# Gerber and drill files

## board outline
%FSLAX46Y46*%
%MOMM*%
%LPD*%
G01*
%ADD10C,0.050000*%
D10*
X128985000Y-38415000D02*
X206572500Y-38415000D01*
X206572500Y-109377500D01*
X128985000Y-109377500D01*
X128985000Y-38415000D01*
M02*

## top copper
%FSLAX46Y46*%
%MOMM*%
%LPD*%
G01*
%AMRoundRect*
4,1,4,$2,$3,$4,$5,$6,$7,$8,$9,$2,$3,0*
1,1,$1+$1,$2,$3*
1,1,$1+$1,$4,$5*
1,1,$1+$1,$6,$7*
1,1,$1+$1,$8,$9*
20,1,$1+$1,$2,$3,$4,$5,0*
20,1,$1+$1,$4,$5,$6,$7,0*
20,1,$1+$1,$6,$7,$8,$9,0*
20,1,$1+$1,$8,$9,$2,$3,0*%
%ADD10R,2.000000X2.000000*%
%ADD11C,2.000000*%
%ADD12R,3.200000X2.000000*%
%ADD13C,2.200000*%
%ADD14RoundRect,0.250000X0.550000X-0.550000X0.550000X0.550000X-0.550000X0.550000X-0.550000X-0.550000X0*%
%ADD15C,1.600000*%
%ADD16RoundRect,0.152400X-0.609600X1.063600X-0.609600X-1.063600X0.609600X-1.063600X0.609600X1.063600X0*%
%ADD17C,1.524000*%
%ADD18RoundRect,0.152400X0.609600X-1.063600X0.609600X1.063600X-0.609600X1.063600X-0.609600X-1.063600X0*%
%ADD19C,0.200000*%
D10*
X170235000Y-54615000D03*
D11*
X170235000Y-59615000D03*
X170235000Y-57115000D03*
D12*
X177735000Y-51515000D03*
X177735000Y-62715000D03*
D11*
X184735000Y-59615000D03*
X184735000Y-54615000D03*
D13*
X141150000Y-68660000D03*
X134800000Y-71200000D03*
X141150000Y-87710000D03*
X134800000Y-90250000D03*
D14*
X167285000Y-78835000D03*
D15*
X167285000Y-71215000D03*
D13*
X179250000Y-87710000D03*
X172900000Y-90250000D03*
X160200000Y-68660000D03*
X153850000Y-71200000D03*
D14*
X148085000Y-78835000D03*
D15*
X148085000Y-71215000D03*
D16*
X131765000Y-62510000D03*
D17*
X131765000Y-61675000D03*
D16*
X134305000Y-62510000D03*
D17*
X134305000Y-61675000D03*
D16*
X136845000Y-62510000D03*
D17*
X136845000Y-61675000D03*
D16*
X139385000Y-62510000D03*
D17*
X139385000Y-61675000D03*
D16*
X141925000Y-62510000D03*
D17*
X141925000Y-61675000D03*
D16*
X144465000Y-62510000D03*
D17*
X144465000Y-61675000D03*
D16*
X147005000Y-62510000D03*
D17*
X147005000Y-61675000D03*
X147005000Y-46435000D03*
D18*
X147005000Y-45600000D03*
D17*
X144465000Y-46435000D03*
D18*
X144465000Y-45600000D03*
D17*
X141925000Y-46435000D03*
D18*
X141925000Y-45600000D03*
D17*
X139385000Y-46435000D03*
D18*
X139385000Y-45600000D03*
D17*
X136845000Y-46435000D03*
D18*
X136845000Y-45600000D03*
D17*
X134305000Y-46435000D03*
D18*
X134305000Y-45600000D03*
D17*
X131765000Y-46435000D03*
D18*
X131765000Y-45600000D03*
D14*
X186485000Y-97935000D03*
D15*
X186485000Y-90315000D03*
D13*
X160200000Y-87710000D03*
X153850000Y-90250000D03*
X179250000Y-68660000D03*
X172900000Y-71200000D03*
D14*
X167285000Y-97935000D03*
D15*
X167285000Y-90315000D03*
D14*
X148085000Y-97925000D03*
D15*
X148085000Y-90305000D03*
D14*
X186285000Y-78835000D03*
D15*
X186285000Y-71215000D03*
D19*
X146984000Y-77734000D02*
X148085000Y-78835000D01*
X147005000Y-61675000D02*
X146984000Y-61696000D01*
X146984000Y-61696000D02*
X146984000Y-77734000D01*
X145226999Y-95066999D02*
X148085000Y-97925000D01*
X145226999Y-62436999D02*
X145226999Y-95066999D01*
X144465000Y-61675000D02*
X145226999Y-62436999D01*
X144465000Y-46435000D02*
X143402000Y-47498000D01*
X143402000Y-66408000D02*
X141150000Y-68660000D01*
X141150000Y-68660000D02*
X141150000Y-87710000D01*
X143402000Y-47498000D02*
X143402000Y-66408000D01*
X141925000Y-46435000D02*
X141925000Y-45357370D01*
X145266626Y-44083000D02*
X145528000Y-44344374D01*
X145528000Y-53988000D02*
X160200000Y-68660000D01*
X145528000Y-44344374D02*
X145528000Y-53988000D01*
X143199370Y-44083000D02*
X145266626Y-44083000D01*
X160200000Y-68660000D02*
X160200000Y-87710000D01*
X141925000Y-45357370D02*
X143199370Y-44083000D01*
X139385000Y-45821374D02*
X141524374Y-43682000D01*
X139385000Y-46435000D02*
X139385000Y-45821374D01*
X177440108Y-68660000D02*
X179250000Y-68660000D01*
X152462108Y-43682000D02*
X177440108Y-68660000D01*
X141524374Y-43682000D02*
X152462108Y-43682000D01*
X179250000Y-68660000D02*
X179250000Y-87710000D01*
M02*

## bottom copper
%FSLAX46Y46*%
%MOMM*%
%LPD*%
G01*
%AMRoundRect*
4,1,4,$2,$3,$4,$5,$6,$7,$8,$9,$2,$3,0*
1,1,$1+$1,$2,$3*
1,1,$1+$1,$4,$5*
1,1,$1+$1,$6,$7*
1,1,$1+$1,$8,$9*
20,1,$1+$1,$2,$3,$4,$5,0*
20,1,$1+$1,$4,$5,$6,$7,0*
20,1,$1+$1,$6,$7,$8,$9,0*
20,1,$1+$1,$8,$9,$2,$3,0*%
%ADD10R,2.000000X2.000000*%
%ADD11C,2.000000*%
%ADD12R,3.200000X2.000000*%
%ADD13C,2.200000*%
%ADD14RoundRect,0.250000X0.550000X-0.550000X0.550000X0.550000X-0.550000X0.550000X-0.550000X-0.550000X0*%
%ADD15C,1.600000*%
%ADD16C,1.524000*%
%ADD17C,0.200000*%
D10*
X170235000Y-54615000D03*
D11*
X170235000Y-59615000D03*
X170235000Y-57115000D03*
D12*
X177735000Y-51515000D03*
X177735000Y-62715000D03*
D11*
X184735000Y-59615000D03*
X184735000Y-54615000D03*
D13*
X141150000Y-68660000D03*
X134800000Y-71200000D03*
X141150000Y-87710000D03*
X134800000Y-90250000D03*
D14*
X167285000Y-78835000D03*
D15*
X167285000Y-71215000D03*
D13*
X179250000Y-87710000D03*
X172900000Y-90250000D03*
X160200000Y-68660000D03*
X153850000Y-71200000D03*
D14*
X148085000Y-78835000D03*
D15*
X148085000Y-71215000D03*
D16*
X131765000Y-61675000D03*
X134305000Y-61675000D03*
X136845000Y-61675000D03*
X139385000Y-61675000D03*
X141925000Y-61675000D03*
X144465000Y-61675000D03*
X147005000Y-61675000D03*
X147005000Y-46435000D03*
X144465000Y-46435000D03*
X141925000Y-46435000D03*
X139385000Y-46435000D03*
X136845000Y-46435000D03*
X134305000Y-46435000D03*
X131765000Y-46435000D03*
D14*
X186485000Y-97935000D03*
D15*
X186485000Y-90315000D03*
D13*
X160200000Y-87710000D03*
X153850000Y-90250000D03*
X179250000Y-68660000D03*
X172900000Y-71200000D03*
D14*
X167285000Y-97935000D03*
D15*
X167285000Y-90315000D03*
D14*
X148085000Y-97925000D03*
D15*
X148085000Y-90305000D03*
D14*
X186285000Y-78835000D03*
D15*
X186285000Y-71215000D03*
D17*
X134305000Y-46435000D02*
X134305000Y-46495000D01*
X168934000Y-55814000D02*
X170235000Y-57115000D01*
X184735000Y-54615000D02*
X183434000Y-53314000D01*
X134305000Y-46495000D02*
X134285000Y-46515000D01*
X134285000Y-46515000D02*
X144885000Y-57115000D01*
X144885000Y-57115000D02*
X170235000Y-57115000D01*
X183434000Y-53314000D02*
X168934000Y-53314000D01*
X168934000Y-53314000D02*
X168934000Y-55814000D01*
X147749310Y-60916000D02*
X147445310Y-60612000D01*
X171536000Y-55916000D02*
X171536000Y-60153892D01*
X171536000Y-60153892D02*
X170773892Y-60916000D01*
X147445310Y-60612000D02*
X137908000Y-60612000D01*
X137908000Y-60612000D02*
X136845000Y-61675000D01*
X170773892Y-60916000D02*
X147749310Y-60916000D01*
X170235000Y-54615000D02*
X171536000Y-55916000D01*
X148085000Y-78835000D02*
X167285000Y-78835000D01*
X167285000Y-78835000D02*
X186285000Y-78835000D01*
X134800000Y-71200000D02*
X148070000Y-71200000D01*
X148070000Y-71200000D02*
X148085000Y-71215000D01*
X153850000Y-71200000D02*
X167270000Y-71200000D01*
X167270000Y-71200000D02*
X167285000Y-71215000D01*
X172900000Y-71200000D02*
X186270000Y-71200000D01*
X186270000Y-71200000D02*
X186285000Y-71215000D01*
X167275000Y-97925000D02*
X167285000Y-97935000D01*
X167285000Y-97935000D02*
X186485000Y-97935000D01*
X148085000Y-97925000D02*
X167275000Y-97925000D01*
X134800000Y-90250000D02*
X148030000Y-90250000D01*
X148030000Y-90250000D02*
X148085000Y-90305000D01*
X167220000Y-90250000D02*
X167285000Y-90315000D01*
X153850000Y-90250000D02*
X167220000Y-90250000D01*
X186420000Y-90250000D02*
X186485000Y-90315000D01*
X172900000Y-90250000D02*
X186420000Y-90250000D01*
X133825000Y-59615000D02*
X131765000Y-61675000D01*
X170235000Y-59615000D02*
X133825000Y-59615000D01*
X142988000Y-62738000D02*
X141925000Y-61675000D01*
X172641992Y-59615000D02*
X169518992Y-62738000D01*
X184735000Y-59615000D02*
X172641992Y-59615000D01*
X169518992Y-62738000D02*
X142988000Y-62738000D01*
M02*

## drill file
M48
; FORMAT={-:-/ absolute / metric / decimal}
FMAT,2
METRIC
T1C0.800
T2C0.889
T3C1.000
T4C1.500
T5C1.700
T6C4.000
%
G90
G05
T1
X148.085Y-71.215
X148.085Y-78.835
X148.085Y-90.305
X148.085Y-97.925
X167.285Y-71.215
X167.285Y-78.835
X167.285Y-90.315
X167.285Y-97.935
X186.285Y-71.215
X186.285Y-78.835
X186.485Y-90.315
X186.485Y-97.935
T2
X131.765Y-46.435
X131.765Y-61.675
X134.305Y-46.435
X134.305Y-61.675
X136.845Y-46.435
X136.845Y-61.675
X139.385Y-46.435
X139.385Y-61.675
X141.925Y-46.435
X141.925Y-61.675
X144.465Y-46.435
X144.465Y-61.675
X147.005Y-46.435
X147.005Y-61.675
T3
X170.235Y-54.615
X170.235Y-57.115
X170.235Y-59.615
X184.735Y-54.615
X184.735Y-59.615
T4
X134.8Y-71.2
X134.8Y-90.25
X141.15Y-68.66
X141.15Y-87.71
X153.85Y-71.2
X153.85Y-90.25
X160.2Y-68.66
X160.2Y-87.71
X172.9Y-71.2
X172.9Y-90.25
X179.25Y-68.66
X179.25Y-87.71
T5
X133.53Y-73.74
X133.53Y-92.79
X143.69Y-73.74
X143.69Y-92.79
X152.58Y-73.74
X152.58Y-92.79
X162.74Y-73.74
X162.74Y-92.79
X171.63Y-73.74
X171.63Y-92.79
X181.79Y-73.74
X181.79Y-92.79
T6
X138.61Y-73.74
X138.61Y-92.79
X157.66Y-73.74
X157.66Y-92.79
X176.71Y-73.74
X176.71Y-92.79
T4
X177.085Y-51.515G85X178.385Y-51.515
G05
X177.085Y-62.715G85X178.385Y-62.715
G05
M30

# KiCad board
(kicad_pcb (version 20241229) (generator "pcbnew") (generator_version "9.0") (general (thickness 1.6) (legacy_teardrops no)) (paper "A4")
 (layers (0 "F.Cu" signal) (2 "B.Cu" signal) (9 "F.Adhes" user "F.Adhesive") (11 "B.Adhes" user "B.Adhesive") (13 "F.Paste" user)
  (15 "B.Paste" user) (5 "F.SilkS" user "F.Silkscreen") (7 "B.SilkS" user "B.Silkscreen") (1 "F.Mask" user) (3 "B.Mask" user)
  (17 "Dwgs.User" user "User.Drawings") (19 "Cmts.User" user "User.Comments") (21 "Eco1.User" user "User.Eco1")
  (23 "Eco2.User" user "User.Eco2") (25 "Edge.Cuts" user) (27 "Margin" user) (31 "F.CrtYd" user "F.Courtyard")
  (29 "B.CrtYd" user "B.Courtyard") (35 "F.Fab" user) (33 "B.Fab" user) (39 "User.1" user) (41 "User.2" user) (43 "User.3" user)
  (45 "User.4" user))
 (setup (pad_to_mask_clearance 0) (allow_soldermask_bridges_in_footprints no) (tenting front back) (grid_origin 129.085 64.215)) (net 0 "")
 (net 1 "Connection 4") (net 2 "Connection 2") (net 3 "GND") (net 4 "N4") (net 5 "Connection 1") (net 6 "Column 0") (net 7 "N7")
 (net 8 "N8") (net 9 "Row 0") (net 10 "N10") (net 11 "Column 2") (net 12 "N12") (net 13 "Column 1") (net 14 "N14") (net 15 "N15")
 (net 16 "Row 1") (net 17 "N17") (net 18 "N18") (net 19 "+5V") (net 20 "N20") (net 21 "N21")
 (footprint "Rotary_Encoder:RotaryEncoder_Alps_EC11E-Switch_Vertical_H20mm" (layer "F.Cu") (at 170.235 54.615)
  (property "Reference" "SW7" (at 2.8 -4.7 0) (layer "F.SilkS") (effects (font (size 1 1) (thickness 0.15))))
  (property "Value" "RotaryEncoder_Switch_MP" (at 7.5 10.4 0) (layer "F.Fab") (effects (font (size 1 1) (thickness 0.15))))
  (pad "A" thru_hole rect (at 0 0) (size 2 2) (drill 1) (layers "*.Cu" "*.Mask") (remove_unused_layers no) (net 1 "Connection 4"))
  (pad "B" thru_hole circle (at 0 5) (size 2 2) (drill 1) (layers "*.Cu" "*.Mask") (remove_unused_layers no) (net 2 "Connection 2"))
  (pad "C" thru_hole circle (at 0 2.5) (size 2 2) (drill 1) (layers "*.Cu" "*.Mask") (remove_unused_layers no) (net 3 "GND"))
  (pad "MP" thru_hole rect (at 7.5 -3.1) (size 3.2 2) (drill oval 2.8 1.5) (layers "*.Cu" "*.Mask") (remove_unused_layers no) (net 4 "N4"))
  (pad "MP" thru_hole rect (at 7.5 8.1) (size 3.2 2) (drill oval 2.8 1.5) (layers "*.Cu" "*.Mask") (remove_unused_layers no) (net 4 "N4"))
  (pad "S1" thru_hole circle (at 14.5 5) (size 2 2) (drill 1) (layers "*.Cu" "*.Mask") (remove_unused_layers no) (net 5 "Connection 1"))
  (pad "S2" thru_hole circle (at 14.5 0) (size 2 2) (drill 1) (layers "*.Cu" "*.Mask") (remove_unused_layers no) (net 3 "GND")))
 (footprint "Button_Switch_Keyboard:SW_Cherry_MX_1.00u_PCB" (layer "F.Cu") (at 141.15 68.66)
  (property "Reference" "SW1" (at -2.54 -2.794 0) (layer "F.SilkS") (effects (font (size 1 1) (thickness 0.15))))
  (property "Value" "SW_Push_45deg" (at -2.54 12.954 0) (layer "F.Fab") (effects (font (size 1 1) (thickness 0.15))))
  (pad "" np_thru_hole circle (at -7.62 5.08) (size 1.7 1.7) (drill 1.7) (layers "*.Cu" "*.Mask"))
  (pad "" np_thru_hole circle (at -2.54 5.08) (size 4 4) (drill 4) (layers "*.Cu" "*.Mask"))
  (pad "" np_thru_hole circle (at 2.54 5.08) (size 1.7 1.7) (drill 1.7) (layers "*.Cu" "*.Mask"))
  (pad "1" thru_hole circle (at 0 0) (size 2.2 2.2) (drill 1.5) (layers "*.Cu" "*.Mask") (remove_unused_layers no) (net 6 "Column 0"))
  (pad "2" thru_hole circle (at -6.35 2.54) (size 2.2 2.2) (drill 1.5) (layers "*.Cu" "*.Mask") (remove_unused_layers no) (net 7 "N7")))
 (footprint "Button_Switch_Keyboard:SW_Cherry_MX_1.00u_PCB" (layer "F.Cu") (at 141.15 87.71)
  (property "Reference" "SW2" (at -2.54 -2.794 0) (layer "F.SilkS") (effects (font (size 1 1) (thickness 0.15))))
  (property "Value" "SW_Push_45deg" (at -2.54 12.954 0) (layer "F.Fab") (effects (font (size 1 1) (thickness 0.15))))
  (pad "" np_thru_hole circle (at -7.62 5.08) (size 1.7 1.7) (drill 1.7) (layers "*.Cu" "*.Mask"))
  (pad "" np_thru_hole circle (at -2.54 5.08) (size 4 4) (drill 4) (layers "*.Cu" "*.Mask"))
  (pad "" np_thru_hole circle (at 2.54 5.08) (size 1.7 1.7) (drill 1.7) (layers "*.Cu" "*.Mask"))
  (pad "1" thru_hole circle (at 0 0) (size 2.2 2.2) (drill 1.5) (layers "*.Cu" "*.Mask") (remove_unused_layers no) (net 6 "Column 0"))
  (pad "2" thru_hole circle (at -6.35 2.54) (size 2.2 2.2) (drill 1.5) (layers "*.Cu" "*.Mask") (remove_unused_layers no) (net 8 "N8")))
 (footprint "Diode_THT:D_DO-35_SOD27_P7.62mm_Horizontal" (layer "F.Cu") (at 167.285 78.835 90)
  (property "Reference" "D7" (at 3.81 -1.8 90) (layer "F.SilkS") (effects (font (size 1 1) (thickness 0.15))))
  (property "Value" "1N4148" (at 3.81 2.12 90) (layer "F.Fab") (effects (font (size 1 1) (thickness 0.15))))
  (pad "1" thru_hole roundrect (at 0 0 90) (size 1.6 1.6) (drill 0.8) (layers "*.Cu" "*.Mask") (remove_unused_layers no)
   (roundrect_rratio 0.15625) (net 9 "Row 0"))
  (pad "2" thru_hole circle (at 7.62 0 90) (size 1.6 1.6) (drill 0.8) (layers "*.Cu" "*.Mask") (remove_unused_layers no) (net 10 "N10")))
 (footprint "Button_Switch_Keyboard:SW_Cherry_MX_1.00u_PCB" (layer "F.Cu") (at 179.25 87.71)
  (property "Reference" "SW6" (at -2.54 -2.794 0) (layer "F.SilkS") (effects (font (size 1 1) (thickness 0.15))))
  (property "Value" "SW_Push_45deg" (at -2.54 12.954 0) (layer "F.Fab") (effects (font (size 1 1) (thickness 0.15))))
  (pad "" np_thru_hole circle (at -7.62 5.08) (size 1.7 1.7) (drill 1.7) (layers "*.Cu" "*.Mask"))
  (pad "" np_thru_hole circle (at -2.54 5.08) (size 4 4) (drill 4) (layers "*.Cu" "*.Mask"))
  (pad "" np_thru_hole circle (at 2.54 5.08) (size 1.7 1.7) (drill 1.7) (layers "*.Cu" "*.Mask"))
  (pad "1" thru_hole circle (at 0 0) (size 2.2 2.2) (drill 1.5) (layers "*.Cu" "*.Mask") (remove_unused_layers no) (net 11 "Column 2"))
  (pad "2" thru_hole circle (at -6.35 2.54) (size 2.2 2.2) (drill 1.5) (layers "*.Cu" "*.Mask") (remove_unused_layers no) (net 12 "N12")))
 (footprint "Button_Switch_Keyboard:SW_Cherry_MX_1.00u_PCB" (layer "F.Cu") (at 160.2 68.66)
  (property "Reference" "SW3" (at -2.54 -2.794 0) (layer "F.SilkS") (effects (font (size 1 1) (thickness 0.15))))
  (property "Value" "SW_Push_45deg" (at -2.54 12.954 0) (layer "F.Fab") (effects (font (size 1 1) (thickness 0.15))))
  (pad "" np_thru_hole circle (at -7.62 5.08) (size 1.7 1.7) (drill 1.7) (layers "*.Cu" "*.Mask"))
  (pad "" np_thru_hole circle (at -2.54 5.08) (size 4 4) (drill 4) (layers "*.Cu" "*.Mask"))
  (pad "" np_thru_hole circle (at 2.54 5.08) (size 1.7 1.7) (drill 1.7) (layers "*.Cu" "*.Mask"))
  (pad "1" thru_hole circle (at 0 0) (size 2.2 2.2) (drill 1.5) (layers "*.Cu" "*.Mask") (remove_unused_layers no) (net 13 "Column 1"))
  (pad "2" thru_hole circle (at -6.35 2.54) (size 2.2 2.2) (drill 1.5) (layers "*.Cu" "*.Mask") (remove_unused_layers no) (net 10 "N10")))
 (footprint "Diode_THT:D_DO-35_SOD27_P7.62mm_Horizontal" (layer "F.Cu") (at 148.085 78.835 90)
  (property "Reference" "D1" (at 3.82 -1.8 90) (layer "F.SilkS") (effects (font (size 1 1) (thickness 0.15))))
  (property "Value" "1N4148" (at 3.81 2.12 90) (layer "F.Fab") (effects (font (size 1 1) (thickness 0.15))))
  (pad "1" thru_hole roundrect (at 0 0 90) (size 1.6 1.6) (drill 0.8) (layers "*.Cu" "*.Mask") (remove_unused_layers no)
   (roundrect_rratio 0.15625) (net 9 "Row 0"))
  (pad "2" thru_hole circle (at 7.62 0 90) (size 1.6 1.6) (drill 0.8) (layers "*.Cu" "*.Mask") (remove_unused_layers no) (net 7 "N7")))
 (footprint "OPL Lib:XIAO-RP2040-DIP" (layer "F.Cu") (at 139.385 54.055 90)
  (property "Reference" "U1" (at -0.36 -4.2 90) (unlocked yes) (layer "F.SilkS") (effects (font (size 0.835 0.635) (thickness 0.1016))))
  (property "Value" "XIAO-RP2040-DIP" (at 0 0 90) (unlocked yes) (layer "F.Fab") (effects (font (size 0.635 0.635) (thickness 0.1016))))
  (pad "1" smd roundrect (at -8.455 -7.62 270) (size 2.432 1.524) (layers "F.Cu" "F.Mask") (roundrect_rratio 0.1) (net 2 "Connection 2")
   (thermal_bridge_angle 45))
  (pad "1" thru_hole circle (at -7.62 -7.62 270) (size 1.524 1.524) (drill 0.889) (layers "*.Cu" "*.Mask") (remove_unused_layers no)
   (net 2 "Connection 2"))
  (pad "2" smd roundrect (at -8.455 -5.08 270) (size 2.432 1.524) (layers "F.Cu" "F.Mask") (roundrect_rratio 0.1) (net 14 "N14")
   (thermal_bridge_angle 45))
  (pad "2" thru_hole circle (at -7.62 -5.08 270) (size 1.524 1.524) (drill 0.889) (layers "*.Cu" "*.Mask") (remove_unused_layers no)
   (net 14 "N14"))
  (pad "3" smd roundrect (at -8.455 -2.54 270) (size 2.432 1.524) (layers "F.Cu" "F.Mask") (roundrect_rratio 0.1) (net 1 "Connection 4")
   (thermal_bridge_angle 45))
  (pad "3" thru_hole circle (at -7.62 -2.54 270) (size 1.524 1.524) (drill 0.889) (layers "*.Cu" "*.Mask") (remove_unused_layers no)
   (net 1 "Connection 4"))
  (pad "4" smd roundrect (at -8.455 0 270) (size 2.432 1.524) (layers "F.Cu" "F.Mask") (roundrect_rratio 0.1) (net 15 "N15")
   (thermal_bridge_angle 45))
  (pad "4" thru_hole circle (at -7.62 0 270) (size 1.524 1.524) (drill 0.889) (layers "*.Cu" "*.Mask") (remove_unused_layers no)
   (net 15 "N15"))
  (pad "5" smd roundrect (at -8.455 2.54 270) (size 2.432 1.524) (layers "F.Cu" "F.Mask") (roundrect_rratio 0.1) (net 5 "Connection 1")
   (thermal_bridge_angle 45))
  (pad "5" thru_hole circle (at -7.62 2.54 270) (size 1.524 1.524) (drill 0.889) (layers "*.Cu" "*.Mask") (remove_unused_layers no)
   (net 5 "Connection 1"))
  (pad "6" smd roundrect (at -8.455 5.08 270) (size 2.432 1.524) (layers "F.Cu" "F.Mask") (roundrect_rratio 0.1) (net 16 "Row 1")
   (thermal_bridge_angle 45))
  (pad "6" thru_hole circle (at -7.62 5.08 270) (size 1.524 1.524) (drill 0.889) (layers "*.Cu" "*.Mask") (remove_unused_layers no)
   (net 16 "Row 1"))
  (pad "7" smd roundrect (at -8.455 7.62 270) (size 2.432 1.524) (layers "F.Cu" "F.Mask") (roundrect_rratio 0.1) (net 9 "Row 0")
   (thermal_bridge_angle 45))
  (pad "7" thru_hole circle (at -7.62 7.62 270) (size 1.524 1.524) (drill 0.889) (layers "*.Cu" "*.Mask") (remove_unused_layers no)
   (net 9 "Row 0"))
  (pad "8" thru_hole circle (at 7.62 7.62 90) (size 1.524 1.524) (drill 0.889) (layers "*.Cu" "*.Mask") (remove_unused_layers no)
   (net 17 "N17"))
  (pad "8" smd roundrect (at 8.455 7.62 90) (size 2.432 1.524) (layers "F.Cu" "F.Mask") (roundrect_rratio 0.1) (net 17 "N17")
   (thermal_bridge_angle 45))
  (pad "9" thru_hole circle (at 7.62 5.08 90) (size 1.524 1.524) (drill 0.889) (layers "*.Cu" "*.Mask") (remove_unused_layers no)
   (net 6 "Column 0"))
  (pad "9" smd roundrect (at 8.455 5.08 90) (size 2.432 1.524) (layers "F.Cu" "F.Mask") (roundrect_rratio 0.1) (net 6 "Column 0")
   (thermal_bridge_angle 45))
  (pad "10" thru_hole circle (at 7.62 2.54 90) (size 1.524 1.524) (drill 0.889) (layers "*.Cu" "*.Mask") (remove_unused_layers no)
   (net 13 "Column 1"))
  (pad "10" smd roundrect (at 8.455 2.54 90) (size 2.432 1.524) (layers "F.Cu" "F.Mask") (roundrect_rratio 0.1) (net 13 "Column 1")
   (thermal_bridge_angle 45))
  (pad "11" thru_hole circle (at 7.62 0 90) (size 1.524 1.524) (drill 0.889) (layers "*.Cu" "*.Mask") (remove_unused_layers no)
   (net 11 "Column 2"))
  (pad "11" smd roundrect (at 8.455 0 90) (size 2.432 1.524) (layers "F.Cu" "F.Mask") (roundrect_rratio 0.1) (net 11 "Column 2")
   (thermal_bridge_angle 45))
  (pad "12" thru_hole circle (at 7.62 -2.54 90) (size 1.524 1.524) (drill 0.889) (layers "*.Cu" "*.Mask") (remove_unused_layers no)
   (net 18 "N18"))
  (pad "12" smd roundrect (at 8.455 -2.54 90) (size 2.432 1.524) (layers "F.Cu" "F.Mask") (roundrect_rratio 0.1) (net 18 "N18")
   (thermal_bridge_angle 45))
  (pad "13" thru_hole circle (at 7.62 -5.08 90) (size 1.524 1.524) (drill 0.889) (layers "*.Cu" "*.Mask") (remove_unused_layers no)
   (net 3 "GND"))
  (pad "13" smd roundrect (at 8.455 -5.08 90) (size 2.432 1.524) (layers "F.Cu" "F.Mask") (roundrect_rratio 0.1) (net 3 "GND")
   (thermal_bridge_angle 45))
  (pad "14" thru_hole circle (at 7.62 -7.62 90) (size 1.524 1.524) (drill 0.889) (layers "*.Cu" "*.Mask") (remove_unused_layers no)
   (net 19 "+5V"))
  (pad "14" smd roundrect (at 8.455 -7.62 90) (size 2.432 1.524) (layers "F.Cu" "F.Mask") (roundrect_rratio 0.1) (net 19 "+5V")
   (thermal_bridge_angle 45)))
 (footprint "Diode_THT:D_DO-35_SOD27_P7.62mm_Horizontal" (layer "F.Cu") (at 186.485 97.935 90)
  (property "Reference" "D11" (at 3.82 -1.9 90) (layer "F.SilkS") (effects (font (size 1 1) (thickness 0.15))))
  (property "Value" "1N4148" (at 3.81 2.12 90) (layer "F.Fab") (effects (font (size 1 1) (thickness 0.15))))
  (pad "1" thru_hole roundrect (at 0 0 90) (size 1.6 1.6) (drill 0.8) (layers "*.Cu" "*.Mask") (remove_unused_layers no)
   (roundrect_rratio 0.15625) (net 16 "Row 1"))
  (pad "2" thru_hole circle (at 7.62 0 90) (size 1.6 1.6) (drill 0.8) (layers "*.Cu" "*.Mask") (remove_unused_layers no) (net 12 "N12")))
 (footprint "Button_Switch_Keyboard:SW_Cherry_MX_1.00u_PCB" (layer "F.Cu") (at 160.2 87.71)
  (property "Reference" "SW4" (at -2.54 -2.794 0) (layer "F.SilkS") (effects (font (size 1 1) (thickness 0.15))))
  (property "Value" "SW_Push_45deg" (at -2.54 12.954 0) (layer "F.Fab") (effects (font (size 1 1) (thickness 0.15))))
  (pad "" np_thru_hole circle (at -7.62 5.08) (size 1.7 1.7) (drill 1.7) (layers "*.Cu" "*.Mask"))
  (pad "" np_thru_hole circle (at -2.54 5.08) (size 4 4) (drill 4) (layers "*.Cu" "*.Mask"))
  (pad "" np_thru_hole circle (at 2.54 5.08) (size 1.7 1.7) (drill 1.7) (layers "*.Cu" "*.Mask"))
  (pad "1" thru_hole circle (at 0 0) (size 2.2 2.2) (drill 1.5) (layers "*.Cu" "*.Mask") (remove_unused_layers no) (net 13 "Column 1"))
  (pad "2" thru_hole circle (at -6.35 2.54) (size 2.2 2.2) (drill 1.5) (layers "*.Cu" "*.Mask") (remove_unused_layers no) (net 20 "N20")))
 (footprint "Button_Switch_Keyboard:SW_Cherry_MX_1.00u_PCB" (layer "F.Cu") (at 179.25 68.66)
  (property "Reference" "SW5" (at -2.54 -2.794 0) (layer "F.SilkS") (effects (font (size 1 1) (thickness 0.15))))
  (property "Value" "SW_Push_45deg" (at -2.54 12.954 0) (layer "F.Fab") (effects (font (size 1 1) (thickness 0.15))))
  (pad "" np_thru_hole circle (at -7.62 5.08) (size 1.7 1.7) (drill 1.7) (layers "*.Cu" "*.Mask"))
  (pad "" np_thru_hole circle (at -2.54 5.08) (size 4 4) (drill 4) (layers "*.Cu" "*.Mask"))
  (pad "" np_thru_hole circle (at 2.54 5.08) (size 1.7 1.7) (drill 1.7) (layers "*.Cu" "*.Mask"))
  (pad "1" thru_hole circle (at 0 0) (size 2.2 2.2) (drill 1.5) (layers "*.Cu" "*.Mask") (remove_unused_layers no) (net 11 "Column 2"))
  (pad "2" thru_hole circle (at -6.35 2.54) (size 2.2 2.2) (drill 1.5) (layers "*.Cu" "*.Mask") (remove_unused_layers no) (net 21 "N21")))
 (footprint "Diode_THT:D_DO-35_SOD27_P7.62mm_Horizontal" (layer "F.Cu") (at 167.285 97.935 90)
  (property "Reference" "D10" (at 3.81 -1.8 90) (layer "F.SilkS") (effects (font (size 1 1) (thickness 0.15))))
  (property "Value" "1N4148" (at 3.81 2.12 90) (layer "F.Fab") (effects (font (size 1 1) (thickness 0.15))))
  (pad "1" thru_hole roundrect (at 0 0 90) (size 1.6 1.6) (drill 0.8) (layers "*.Cu" "*.Mask") (remove_unused_layers no)
   (roundrect_rratio 0.15625) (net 16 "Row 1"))
  (pad "2" thru_hole circle (at 7.62 0 90) (size 1.6 1.6) (drill 0.8) (layers "*.Cu" "*.Mask") (remove_unused_layers no) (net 20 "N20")))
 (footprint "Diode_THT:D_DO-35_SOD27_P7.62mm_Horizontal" (layer "F.Cu") (at 148.085 97.925 90)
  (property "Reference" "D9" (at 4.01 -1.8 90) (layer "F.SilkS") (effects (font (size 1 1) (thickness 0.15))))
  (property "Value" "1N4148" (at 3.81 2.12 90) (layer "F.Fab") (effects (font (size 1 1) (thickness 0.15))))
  (pad "1" thru_hole roundrect (at 0 0 90) (size 1.6 1.6) (drill 0.8) (layers "*.Cu" "*.Mask") (remove_unused_layers no)
   (roundrect_rratio 0.15625) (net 16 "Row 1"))
  (pad "2" thru_hole circle (at 7.62 0 90) (size 1.6 1.6) (drill 0.8) (layers "*.Cu" "*.Mask") (remove_unused_layers no) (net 8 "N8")))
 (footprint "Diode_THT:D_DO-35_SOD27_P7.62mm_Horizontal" (layer "F.Cu") (at 186.285 78.835 90)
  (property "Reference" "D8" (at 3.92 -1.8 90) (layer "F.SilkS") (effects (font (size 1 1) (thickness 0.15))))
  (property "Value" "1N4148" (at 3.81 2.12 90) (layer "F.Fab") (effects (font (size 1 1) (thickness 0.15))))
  (pad "1" thru_hole roundrect (at 0 0 90) (size 1.6 1.6) (drill 0.8) (layers "*.Cu" "*.Mask") (remove_unused_layers no)
   (roundrect_rratio 0.15625) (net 9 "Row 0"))
  (pad "2" thru_hole circle (at 7.62 0 90) (size 1.6 1.6) (drill 0.8) (layers "*.Cu" "*.Mask") (remove_unused_layers no) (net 21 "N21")))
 (gr_rect (start 128.985 38.415) (end 206.5725 109.3775) (stroke (width 0.05) (type default)) (fill no) (layer "Edge.Cuts"))
 (segment (start 134.305 46.435) (end 134.305 46.495) (width 0.2) (layer "B.Cu") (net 3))
 (segment (start 168.934 55.814) (end 170.235 57.115) (width 0.2) (layer "B.Cu") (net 3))
 (segment (start 184.735 54.615) (end 183.434 53.314) (width 0.2) (layer "B.Cu") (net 3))
 (segment (start 134.305 46.495) (end 134.285 46.515) (width 0.2) (layer "B.Cu") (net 3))
 (segment (start 134.285 46.515) (end 144.885 57.115) (width 0.2) (layer "B.Cu") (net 3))
 (segment (start 144.885 57.115) (end 170.235 57.115) (width 0.2) (layer "B.Cu") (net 3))
 (segment (start 183.434 53.314) (end 168.934 53.314) (width 0.2) (layer "B.Cu") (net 3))
 (segment (start 168.934 53.314) (end 168.934 55.814) (width 0.2) (layer "B.Cu") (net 3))
 (segment (start 147.74931 60.916) (end 147.44531 60.612) (width 0.2) (layer "B.Cu") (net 1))
 (segment (start 171.536 55.916) (end 171.536 60.153892) (width 0.2) (layer "B.Cu") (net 1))
 (segment (start 171.536 60.153892) (end 170.773892 60.916) (width 0.2) (layer "B.Cu") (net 1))
 (segment (start 147.44531 60.612) (end 137.908 60.612) (width 0.2) (layer "B.Cu") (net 1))
 (segment (start 137.908 60.612) (end 136.845 61.675) (width 0.2) (layer "B.Cu") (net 1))
 (segment (start 170.773892 60.916) (end 147.74931 60.916) (width 0.2) (layer "B.Cu") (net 1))
 (segment (start 170.235 54.615) (end 171.536 55.916) (width 0.2) (layer "B.Cu") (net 1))
 (segment (start 146.984 77.734) (end 148.085 78.835) (width 0.2) (layer "F.Cu") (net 9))
 (segment (start 147.005 61.675) (end 146.984 61.696) (width 0.2) (layer "F.Cu") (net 9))
 (segment (start 146.984 61.696) (end 146.984 77.734) (width 0.2) (layer "F.Cu") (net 9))
 (segment (start 148.085 78.835) (end 167.285 78.835) (width 0.2) (layer "B.Cu") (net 9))
 (segment (start 167.285 78.835) (end 186.285 78.835) (width 0.2) (layer "B.Cu") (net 9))
 (segment (start 134.8 71.2) (end 148.07 71.2) (width 0.2) (layer "B.Cu") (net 7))
 (segment (start 148.07 71.2) (end 148.085 71.215) (width 0.2) (layer "B.Cu") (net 7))
 (segment (start 153.85 71.2) (end 167.27 71.2) (width 0.2) (layer "B.Cu") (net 10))
 (segment (start 167.27 71.2) (end 167.285 71.215) (width 0.2) (layer "B.Cu") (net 10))
 (segment (start 172.9 71.2) (end 186.27 71.2) (width 0.2) (layer "B.Cu") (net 21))
 (segment (start 186.27 71.2) (end 186.285 71.215) (width 0.2) (layer "B.Cu") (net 21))
 (segment (start 145.226999 95.066999) (end 148.085 97.925) (width 0.2) (layer "F.Cu") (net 16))
 (segment (start 145.226999 62.436999) (end 145.226999 95.066999) (width 0.2) (layer "F.Cu") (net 16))
 (segment (start 144.465 61.675) (end 145.226999 62.436999) (width 0.2) (layer "F.Cu") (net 16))
 (segment (start 167.275 97.925) (end 167.285 97.935) (width 0.2) (layer "B.Cu") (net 16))
 (segment (start 167.285 97.935) (end 186.485 97.935) (width 0.2) (layer "B.Cu") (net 16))
 (segment (start 148.085 97.925) (end 167.275 97.925) (width 0.2) (layer "B.Cu") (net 16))
 (segment (start 134.8 90.25) (end 148.03 90.25) (width 0.2) (layer "B.Cu") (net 8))
 (segment (start 148.03 90.25) (end 148.085 90.305) (width 0.2) (layer "B.Cu") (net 8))
 (segment (start 167.22 90.25) (end 167.285 90.315) (width 0.2) (layer "B.Cu") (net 20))
 (segment (start 153.85 90.25) (end 167.22 90.25) (width 0.2) (layer "B.Cu") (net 20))
 (segment (start 186.42 90.25) (end 186.485 90.315) (width 0.2) (layer "B.Cu") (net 12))
 (segment (start 172.9 90.25) (end 186.42 90.25) (width 0.2) (layer "B.Cu") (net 12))
 (segment (start 144.465 46.435) (end 143.402 47.498) (width 0.2) (layer "F.Cu") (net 6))
 (segment (start 143.402 66.408) (end 141.15 68.66) (width 0.2) (layer "F.Cu") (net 6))
 (segment (start 141.15 68.66) (end 141.15 87.71) (width 0.2) (layer "F.Cu") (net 6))
 (segment (start 143.402 47.498) (end 143.402 66.408) (width 0.2) (layer "F.Cu") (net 6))
 (segment (start 141.925 46.435) (end 141.925 45.35737) (width 0.2) (layer "F.Cu") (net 13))
 (segment (start 145.266626 44.083) (end 145.528 44.344374) (width 0.2) (layer "F.Cu") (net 13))
 (segment (start 145.528 53.988) (end 160.2 68.66) (width 0.2) (layer "F.Cu") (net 13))
 (segment (start 145.528 44.344374) (end 145.528 53.988) (width 0.2) (layer "F.Cu") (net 13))
 (segment (start 143.19937 44.083) (end 145.266626 44.083) (width 0.2) (layer "F.Cu") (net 13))
 (segment (start 160.2 68.66) (end 160.2 87.71) (width 0.2) (layer "F.Cu") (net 13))
 (segment (start 141.925 45.35737) (end 143.19937 44.083) (width 0.2) (layer "F.Cu") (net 13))
 (segment (start 139.385 45.821374) (end 141.524374 43.682) (width 0.2) (layer "F.Cu") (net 11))
 (segment (start 139.385 46.435) (end 139.385 45.821374) (width 0.2) (layer "F.Cu") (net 11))
 (segment (start 177.440108 68.66) (end 179.25 68.66) (width 0.2) (layer "F.Cu") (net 11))
 (segment (start 152.462108 43.682) (end 177.440108 68.66) (width 0.2) (layer "F.Cu") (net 11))
 (segment (start 141.524374 43.682) (end 152.462108 43.682) (width 0.2) (layer "F.Cu") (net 11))
 (segment (start 179.25 68.66) (end 179.25 87.71) (width 0.2) (layer "F.Cu") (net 11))
 (segment (start 133.825 59.615) (end 131.765 61.675) (width 0.2) (layer "B.Cu") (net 2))
 (segment (start 170.235 59.615) (end 133.825 59.615) (width 0.2) (layer "B.Cu") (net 2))
 (segment (start 142.988 62.738) (end 141.925 61.675) (width 0.2) (layer "B.Cu") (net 5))
 (segment (start 172.641992 59.615) (end 169.518992 62.738) (width 0.2) (layer "B.Cu") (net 5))
 (segment (start 184.735 59.615) (end 172.641992 59.615) (width 0.2) (layer "B.Cu") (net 5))
 (segment (start 169.518992 62.738) (end 142.988 62.738) (width 0.2) (layer "B.Cu") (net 5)))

